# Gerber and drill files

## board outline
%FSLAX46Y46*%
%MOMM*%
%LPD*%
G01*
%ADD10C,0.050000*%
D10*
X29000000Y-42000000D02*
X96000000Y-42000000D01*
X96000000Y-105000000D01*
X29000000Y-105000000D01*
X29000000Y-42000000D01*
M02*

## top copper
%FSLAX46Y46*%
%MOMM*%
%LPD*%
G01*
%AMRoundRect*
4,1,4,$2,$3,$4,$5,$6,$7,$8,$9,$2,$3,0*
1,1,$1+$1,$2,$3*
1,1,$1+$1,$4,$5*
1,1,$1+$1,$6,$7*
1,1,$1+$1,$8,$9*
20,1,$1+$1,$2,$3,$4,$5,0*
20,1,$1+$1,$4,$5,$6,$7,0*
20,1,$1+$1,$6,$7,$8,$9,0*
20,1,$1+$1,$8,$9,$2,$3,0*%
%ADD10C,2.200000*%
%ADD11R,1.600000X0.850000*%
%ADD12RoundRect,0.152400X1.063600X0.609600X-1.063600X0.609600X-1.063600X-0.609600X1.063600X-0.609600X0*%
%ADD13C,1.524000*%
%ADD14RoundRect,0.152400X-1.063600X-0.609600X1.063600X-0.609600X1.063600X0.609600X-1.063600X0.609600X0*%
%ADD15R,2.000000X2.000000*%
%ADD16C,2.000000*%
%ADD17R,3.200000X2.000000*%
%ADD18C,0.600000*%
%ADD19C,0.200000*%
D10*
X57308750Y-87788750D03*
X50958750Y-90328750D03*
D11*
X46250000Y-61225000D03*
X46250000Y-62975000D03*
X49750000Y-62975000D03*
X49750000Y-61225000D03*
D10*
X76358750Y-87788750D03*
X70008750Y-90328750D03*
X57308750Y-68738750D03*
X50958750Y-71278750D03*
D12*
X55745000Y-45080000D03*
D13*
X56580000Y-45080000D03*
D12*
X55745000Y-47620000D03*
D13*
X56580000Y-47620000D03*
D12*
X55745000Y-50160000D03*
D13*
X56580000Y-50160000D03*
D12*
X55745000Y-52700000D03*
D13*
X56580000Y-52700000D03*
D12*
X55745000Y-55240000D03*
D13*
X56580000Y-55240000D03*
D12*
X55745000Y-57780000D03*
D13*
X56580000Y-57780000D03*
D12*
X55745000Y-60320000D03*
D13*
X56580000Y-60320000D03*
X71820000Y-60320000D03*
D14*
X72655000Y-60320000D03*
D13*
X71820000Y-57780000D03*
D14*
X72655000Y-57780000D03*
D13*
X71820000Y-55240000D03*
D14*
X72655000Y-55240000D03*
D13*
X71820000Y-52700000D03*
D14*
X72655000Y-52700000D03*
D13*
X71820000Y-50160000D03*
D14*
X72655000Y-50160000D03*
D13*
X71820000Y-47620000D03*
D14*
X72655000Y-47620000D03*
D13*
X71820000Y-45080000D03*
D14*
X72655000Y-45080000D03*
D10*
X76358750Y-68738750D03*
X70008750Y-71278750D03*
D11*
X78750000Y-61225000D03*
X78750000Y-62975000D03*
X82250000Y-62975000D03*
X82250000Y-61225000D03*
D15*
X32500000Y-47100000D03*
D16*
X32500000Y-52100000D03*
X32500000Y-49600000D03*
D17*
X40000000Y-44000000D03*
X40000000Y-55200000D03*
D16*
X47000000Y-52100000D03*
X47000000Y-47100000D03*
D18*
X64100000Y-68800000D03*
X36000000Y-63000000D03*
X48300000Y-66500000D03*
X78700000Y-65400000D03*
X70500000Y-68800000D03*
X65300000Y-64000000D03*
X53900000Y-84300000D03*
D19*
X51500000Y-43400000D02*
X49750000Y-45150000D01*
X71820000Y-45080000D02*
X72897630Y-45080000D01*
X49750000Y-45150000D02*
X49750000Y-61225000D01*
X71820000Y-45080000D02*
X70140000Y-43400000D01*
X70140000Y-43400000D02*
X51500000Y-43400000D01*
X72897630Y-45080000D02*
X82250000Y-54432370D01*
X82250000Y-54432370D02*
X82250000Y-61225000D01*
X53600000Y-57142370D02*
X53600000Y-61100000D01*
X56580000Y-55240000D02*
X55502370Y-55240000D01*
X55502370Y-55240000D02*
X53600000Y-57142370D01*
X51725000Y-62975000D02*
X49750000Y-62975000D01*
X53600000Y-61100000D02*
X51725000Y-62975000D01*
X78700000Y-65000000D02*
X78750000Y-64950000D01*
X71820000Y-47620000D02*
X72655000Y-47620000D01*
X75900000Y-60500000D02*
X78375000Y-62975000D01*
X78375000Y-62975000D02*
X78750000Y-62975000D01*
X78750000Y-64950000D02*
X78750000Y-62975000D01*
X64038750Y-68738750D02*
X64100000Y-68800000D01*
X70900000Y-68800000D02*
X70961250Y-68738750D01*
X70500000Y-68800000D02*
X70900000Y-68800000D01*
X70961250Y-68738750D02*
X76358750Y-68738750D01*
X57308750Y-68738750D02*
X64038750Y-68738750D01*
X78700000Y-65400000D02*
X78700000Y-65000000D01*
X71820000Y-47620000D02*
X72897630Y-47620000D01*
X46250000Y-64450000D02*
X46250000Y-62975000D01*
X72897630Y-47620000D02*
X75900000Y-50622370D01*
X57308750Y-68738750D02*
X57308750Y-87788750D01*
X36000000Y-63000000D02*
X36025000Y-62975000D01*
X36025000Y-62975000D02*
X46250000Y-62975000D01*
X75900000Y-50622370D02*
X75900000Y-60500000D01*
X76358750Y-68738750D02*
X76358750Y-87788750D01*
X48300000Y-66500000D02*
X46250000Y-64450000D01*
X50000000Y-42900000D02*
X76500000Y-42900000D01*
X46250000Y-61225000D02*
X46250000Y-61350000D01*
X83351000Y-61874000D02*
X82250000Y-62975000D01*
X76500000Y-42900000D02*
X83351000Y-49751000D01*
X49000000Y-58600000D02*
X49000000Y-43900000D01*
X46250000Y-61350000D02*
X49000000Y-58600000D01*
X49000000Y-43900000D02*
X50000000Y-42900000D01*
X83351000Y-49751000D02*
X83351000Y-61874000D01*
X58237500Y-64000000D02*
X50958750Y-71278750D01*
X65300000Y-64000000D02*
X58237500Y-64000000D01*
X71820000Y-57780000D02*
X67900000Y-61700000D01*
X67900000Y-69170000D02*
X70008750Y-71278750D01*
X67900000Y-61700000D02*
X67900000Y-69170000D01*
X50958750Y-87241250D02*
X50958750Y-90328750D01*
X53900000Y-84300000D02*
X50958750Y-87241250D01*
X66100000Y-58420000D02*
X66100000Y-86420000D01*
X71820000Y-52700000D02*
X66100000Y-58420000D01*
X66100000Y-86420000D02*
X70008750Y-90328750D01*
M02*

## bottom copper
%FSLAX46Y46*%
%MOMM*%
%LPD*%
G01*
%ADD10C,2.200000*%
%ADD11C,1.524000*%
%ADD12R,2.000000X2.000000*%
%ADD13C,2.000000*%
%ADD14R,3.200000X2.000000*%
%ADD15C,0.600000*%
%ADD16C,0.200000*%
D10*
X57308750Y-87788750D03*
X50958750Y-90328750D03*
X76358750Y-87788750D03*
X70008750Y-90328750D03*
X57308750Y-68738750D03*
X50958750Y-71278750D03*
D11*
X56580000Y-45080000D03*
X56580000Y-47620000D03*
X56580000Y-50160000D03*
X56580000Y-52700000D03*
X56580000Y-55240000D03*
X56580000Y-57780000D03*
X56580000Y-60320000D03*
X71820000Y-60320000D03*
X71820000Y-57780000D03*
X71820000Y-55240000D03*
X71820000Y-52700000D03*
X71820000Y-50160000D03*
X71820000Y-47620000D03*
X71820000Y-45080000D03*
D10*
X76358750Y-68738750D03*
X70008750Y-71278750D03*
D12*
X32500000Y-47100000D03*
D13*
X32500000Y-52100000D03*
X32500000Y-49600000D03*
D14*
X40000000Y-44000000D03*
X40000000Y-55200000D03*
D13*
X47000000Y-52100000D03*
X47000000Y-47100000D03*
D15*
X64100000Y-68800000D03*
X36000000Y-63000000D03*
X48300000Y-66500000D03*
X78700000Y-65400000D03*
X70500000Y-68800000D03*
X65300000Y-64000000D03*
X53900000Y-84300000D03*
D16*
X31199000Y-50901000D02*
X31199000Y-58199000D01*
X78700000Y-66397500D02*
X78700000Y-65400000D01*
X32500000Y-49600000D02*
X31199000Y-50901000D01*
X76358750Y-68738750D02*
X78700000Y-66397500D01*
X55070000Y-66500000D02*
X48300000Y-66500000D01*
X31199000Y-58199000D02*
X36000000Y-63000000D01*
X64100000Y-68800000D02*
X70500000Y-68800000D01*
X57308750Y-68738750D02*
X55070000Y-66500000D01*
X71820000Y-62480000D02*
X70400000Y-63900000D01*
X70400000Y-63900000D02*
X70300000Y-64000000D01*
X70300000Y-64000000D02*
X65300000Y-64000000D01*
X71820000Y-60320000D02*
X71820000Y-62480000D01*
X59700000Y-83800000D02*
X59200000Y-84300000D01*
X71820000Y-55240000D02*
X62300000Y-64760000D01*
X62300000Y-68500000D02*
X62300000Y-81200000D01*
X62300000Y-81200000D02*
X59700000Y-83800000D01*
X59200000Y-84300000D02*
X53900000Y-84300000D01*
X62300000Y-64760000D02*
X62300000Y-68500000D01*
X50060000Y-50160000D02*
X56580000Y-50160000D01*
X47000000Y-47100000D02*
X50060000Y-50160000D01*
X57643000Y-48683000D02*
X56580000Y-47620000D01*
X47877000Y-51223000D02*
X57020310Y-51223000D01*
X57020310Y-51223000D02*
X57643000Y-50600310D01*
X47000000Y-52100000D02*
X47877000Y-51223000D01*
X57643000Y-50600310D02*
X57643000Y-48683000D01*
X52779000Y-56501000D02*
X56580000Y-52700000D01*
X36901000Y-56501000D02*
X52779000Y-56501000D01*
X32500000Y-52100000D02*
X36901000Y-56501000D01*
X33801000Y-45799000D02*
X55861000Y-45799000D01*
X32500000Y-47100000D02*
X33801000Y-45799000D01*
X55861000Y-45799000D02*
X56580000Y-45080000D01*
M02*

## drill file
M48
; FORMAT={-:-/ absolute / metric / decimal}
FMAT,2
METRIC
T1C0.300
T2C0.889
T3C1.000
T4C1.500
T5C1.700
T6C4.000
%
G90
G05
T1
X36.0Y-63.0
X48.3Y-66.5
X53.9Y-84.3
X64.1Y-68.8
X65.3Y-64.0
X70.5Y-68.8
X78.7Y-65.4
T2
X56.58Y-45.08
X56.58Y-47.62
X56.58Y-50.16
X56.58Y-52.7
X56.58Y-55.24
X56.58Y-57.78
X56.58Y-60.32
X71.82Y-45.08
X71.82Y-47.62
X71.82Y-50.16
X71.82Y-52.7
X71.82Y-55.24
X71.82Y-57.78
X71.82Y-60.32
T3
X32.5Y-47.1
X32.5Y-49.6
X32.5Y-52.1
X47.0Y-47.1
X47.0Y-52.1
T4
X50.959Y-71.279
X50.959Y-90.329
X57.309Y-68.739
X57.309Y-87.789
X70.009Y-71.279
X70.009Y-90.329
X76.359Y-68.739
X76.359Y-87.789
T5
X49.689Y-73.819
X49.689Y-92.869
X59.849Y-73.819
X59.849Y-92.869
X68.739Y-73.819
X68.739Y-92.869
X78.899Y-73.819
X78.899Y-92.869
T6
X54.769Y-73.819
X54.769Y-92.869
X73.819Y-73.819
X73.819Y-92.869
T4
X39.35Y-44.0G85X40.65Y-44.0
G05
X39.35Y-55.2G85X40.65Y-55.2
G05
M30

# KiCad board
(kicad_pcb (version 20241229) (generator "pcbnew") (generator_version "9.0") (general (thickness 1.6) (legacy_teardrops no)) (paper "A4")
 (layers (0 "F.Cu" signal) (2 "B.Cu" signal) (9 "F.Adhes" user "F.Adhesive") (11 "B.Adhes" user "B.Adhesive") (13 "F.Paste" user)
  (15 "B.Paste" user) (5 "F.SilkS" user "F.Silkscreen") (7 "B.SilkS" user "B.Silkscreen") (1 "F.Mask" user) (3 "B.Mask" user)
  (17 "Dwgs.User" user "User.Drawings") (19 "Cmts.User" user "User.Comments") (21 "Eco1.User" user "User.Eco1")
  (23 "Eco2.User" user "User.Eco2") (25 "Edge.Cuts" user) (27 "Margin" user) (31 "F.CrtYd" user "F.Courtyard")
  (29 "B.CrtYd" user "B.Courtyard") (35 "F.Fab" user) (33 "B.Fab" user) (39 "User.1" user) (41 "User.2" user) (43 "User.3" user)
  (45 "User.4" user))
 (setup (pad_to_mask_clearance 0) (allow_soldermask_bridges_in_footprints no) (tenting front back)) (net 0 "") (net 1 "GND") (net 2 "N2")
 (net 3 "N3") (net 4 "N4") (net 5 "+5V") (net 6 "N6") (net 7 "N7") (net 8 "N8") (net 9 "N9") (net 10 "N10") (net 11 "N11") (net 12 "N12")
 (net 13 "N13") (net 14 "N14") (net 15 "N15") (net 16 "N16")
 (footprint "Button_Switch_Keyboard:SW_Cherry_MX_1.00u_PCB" (layer "F.Cu") (at 57.30875 87.78875)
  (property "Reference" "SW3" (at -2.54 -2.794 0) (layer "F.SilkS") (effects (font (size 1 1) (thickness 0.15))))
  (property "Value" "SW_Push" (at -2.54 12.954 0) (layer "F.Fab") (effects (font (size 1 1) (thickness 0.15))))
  (pad "" np_thru_hole circle (at -7.62 5.08) (size 1.7 1.7) (drill 1.7) (layers "*.Cu" "*.Mask"))
  (pad "" np_thru_hole circle (at -2.54 5.08) (size 4 4) (drill 4) (layers "*.Cu" "*.Mask"))
  (pad "" np_thru_hole circle (at 2.54 5.08) (size 1.7 1.7) (drill 1.7) (layers "*.Cu" "*.Mask"))
  (pad "1" thru_hole circle (at 0 0) (size 2.2 2.2) (drill 1.5) (layers "*.Cu" "*.Mask") (remove_unused_layers no) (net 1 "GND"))
  (pad "2" thru_hole circle (at -6.35 2.54) (size 2.2 2.2) (drill 1.5) (layers "*.Cu" "*.Mask") (remove_unused_layers no) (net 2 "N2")))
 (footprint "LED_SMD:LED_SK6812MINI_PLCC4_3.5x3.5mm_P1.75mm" (layer "F.Cu") (at 48 62.1)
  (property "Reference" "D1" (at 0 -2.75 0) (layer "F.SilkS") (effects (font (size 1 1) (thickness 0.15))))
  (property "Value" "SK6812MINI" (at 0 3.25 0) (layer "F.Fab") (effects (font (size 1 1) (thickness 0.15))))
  (pad "1" smd rect (at -1.75 -0.875) (size 1.6 0.85) (layers "F.Cu" "F.Mask" "F.Paste") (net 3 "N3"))
  (pad "2" smd rect (at -1.75 0.875) (size 1.6 0.85) (layers "F.Cu" "F.Mask" "F.Paste") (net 1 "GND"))
  (pad "3" smd rect (at 1.75 0.875) (size 1.6 0.85) (layers "F.Cu" "F.Mask" "F.Paste") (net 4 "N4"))
  (pad "4" smd rect (at 1.75 -0.875) (size 1.6 0.85) (layers "F.Cu" "F.Mask" "F.Paste") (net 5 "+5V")))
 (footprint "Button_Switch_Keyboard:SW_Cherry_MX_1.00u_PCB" (layer "F.Cu") (at 76.35875 87.78875)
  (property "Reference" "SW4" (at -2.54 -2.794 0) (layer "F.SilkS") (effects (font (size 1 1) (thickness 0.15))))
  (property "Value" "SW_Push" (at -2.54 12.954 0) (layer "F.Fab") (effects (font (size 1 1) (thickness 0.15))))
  (pad "" np_thru_hole circle (at -7.62 5.08) (size 1.7 1.7) (drill 1.7) (layers "*.Cu" "*.Mask"))
  (pad "" np_thru_hole circle (at -2.54 5.08) (size 4 4) (drill 4) (layers "*.Cu" "*.Mask"))
  (pad "" np_thru_hole circle (at 2.54 5.08) (size 1.7 1.7) (drill 1.7) (layers "*.Cu" "*.Mask"))
  (pad "1" thru_hole circle (at 0 0) (size 2.2 2.2) (drill 1.5) (layers "*.Cu" "*.Mask") (remove_unused_layers no) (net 1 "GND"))
  (pad "2" thru_hole circle (at -6.35 2.54) (size 2.2 2.2) (drill 1.5) (layers "*.Cu" "*.Mask") (remove_unused_layers no) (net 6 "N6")))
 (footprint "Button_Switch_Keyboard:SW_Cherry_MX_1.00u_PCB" (layer "F.Cu") (at 57.30875 68.73875)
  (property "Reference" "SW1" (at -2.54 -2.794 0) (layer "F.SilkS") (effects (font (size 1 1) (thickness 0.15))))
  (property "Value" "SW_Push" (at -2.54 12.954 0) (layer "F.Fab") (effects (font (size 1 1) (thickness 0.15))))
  (pad "" np_thru_hole circle (at -7.62 5.08) (size 1.7 1.7) (drill 1.7) (layers "*.Cu" "*.Mask"))
  (pad "" np_thru_hole circle (at -2.54 5.08) (size 4 4) (drill 4) (layers "*.Cu" "*.Mask"))
  (pad "" np_thru_hole circle (at 2.54 5.08) (size 1.7 1.7) (drill 1.7) (layers "*.Cu" "*.Mask"))
  (pad "1" thru_hole circle (at 0 0) (size 2.2 2.2) (drill 1.5) (layers "*.Cu" "*.Mask") (remove_unused_layers no) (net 1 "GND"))
  (pad "2" thru_hole circle (at -6.35 2.54) (size 2.2 2.2) (drill 1.5) (layers "*.Cu" "*.Mask") (remove_unused_layers no) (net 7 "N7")))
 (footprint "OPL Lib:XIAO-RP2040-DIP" (layer "F.Cu") (at 64.2 52.7)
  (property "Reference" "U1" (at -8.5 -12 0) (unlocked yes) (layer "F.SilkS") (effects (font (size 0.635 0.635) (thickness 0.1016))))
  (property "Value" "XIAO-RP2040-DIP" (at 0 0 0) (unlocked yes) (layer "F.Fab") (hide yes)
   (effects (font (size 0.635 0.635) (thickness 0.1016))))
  (pad "1" smd roundrect (at -8.455 -7.62 180) (size 2.432 1.524) (layers "F.Cu" "F.Mask") (roundrect_rratio 0.1) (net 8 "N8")
   (thermal_bridge_angle 45))
  (pad "1" thru_hole circle (at -7.62 -7.62 180) (size 1.524 1.524) (drill 0.889) (layers "*.Cu" "*.Mask") (remove_unused_layers no)
   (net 8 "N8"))
  (pad "2" smd roundrect (at -8.455 -5.08 180) (size 2.432 1.524) (layers "F.Cu" "F.Mask") (roundrect_rratio 0.1) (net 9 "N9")
   (thermal_bridge_angle 45))
  (pad "2" thru_hole circle (at -7.62 -5.08 180) (size 1.524 1.524) (drill 0.889) (layers "*.Cu" "*.Mask") (remove_unused_layers no)
   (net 9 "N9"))
  (pad "3" smd roundrect (at -8.455 -2.54 180) (size 2.432 1.524) (layers "F.Cu" "F.Mask") (roundrect_rratio 0.1) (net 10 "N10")
   (thermal_bridge_angle 45))
  (pad "3" thru_hole circle (at -7.62 -2.54 180) (size 1.524 1.524) (drill 0.889) (layers "*.Cu" "*.Mask") (remove_unused_layers no)
   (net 10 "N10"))
  (pad "4" smd roundrect (at -8.455 0 180) (size 2.432 1.524) (layers "F.Cu" "F.Mask") (roundrect_rratio 0.1) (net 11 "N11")
   (thermal_bridge_angle 45))
  (pad "4" thru_hole circle (at -7.62 0 180) (size 1.524 1.524) (drill 0.889) (layers "*.Cu" "*.Mask") (remove_unused_layers no)
   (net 11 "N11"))
  (pad "5" smd roundrect (at -8.455 2.54 180) (size 2.432 1.524) (layers "F.Cu" "F.Mask") (roundrect_rratio 0.1) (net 4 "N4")
   (thermal_bridge_angle 45))
  (pad "5" thru_hole circle (at -7.62 2.54 180) (size 1.524 1.524) (drill 0.889) (layers "*.Cu" "*.Mask") (remove_unused_layers no)
   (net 4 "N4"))
  (pad "6" smd roundrect (at -8.455 5.08 180) (size 2.432 1.524) (layers "F.Cu" "F.Mask") (roundrect_rratio 0.1) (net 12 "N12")
   (thermal_bridge_angle 45))
  (pad "6" thru_hole circle (at -7.62 5.08 180) (size 1.524 1.524) (drill 0.889) (layers "*.Cu" "*.Mask") (remove_unused_layers no)
   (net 12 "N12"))
  (pad "7" smd roundrect (at -8.455 7.62 180) (size 2.432 1.524) (layers "F.Cu" "F.Mask") (roundrect_rratio 0.1) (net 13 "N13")
   (thermal_bridge_angle 45))
  (pad "7" thru_hole circle (at -7.62 7.62 180) (size 1.524 1.524) (drill 0.889) (layers "*.Cu" "*.Mask") (remove_unused_layers no)
   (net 13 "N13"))
  (pad "8" thru_hole circle (at 7.62 7.62) (size 1.524 1.524) (drill 0.889) (layers "*.Cu" "*.Mask") (remove_unused_layers no) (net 7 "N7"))
  (pad "8" smd roundrect (at 8.455 7.62) (size 2.432 1.524) (layers "F.Cu" "F.Mask") (roundrect_rratio 0.1) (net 7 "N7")
   (thermal_bridge_angle 45))
  (pad "9" thru_hole circle (at 7.62 5.08) (size 1.524 1.524) (drill 0.889) (layers "*.Cu" "*.Mask") (remove_unused_layers no)
   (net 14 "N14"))
  (pad "9" smd roundrect (at 8.455 5.08) (size 2.432 1.524) (layers "F.Cu" "F.Mask") (roundrect_rratio 0.1) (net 14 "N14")
   (thermal_bridge_angle 45))
  (pad "10" thru_hole circle (at 7.62 2.54) (size 1.524 1.524) (drill 0.889) (layers "*.Cu" "*.Mask") (remove_unused_layers no) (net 2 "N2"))
  (pad "10" smd roundrect (at 8.455 2.54) (size 2.432 1.524) (layers "F.Cu" "F.Mask") (roundrect_rratio 0.1) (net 2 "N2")
   (thermal_bridge_angle 45))
  (pad "11" thru_hole circle (at 7.62 0) (size 1.524 1.524) (drill 0.889) (layers "*.Cu" "*.Mask") (remove_unused_layers no) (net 6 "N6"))
  (pad "11" smd roundrect (at 8.455 0) (size 2.432 1.524) (layers "F.Cu" "F.Mask") (roundrect_rratio 0.1) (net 6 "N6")
   (thermal_bridge_angle 45))
  (pad "12" thru_hole circle (at 7.62 -2.54) (size 1.524 1.524) (drill 0.889) (layers "*.Cu" "*.Mask") (remove_unused_layers no)
   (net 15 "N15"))
  (pad "12" smd roundrect (at 8.455 -2.54) (size 2.432 1.524) (layers "F.Cu" "F.Mask") (roundrect_rratio 0.1) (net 15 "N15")
   (thermal_bridge_angle 45))
  (pad "13" thru_hole circle (at 7.62 -5.08) (size 1.524 1.524) (drill 0.889) (layers "*.Cu" "*.Mask") (remove_unused_layers no)
   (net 1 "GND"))
  (pad "13" smd roundrect (at 8.455 -5.08) (size 2.432 1.524) (layers "F.Cu" "F.Mask") (roundrect_rratio 0.1) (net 1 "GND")
   (thermal_bridge_angle 45))
  (pad "14" thru_hole circle (at 7.62 -7.62) (size 1.524 1.524) (drill 0.889) (layers "*.Cu" "*.Mask") (remove_unused_layers no)
   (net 5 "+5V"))
  (pad "14" smd roundrect (at 8.455 -7.62) (size 2.432 1.524) (layers "F.Cu" "F.Mask") (roundrect_rratio 0.1) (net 5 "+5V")
   (thermal_bridge_angle 45)))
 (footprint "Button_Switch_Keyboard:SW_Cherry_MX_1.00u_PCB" (layer "F.Cu") (at 76.35875 68.73875)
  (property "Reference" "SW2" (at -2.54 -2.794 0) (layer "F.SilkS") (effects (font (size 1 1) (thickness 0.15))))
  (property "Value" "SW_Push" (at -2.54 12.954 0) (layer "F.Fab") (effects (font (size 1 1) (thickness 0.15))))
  (pad "" np_thru_hole circle (at -7.62 5.08) (size 1.7 1.7) (drill 1.7) (layers "*.Cu" "*.Mask"))
  (pad "" np_thru_hole circle (at -2.54 5.08) (size 4 4) (drill 4) (layers "*.Cu" "*.Mask"))
  (pad "" np_thru_hole circle (at 2.54 5.08) (size 1.7 1.7) (drill 1.7) (layers "*.Cu" "*.Mask"))
  (pad "1" thru_hole circle (at 0 0) (size 2.2 2.2) (drill 1.5) (layers "*.Cu" "*.Mask") (remove_unused_layers no) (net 1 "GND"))
  (pad "2" thru_hole circle (at -6.35 2.54) (size 2.2 2.2) (drill 1.5) (layers "*.Cu" "*.Mask") (remove_unused_layers no) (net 14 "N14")))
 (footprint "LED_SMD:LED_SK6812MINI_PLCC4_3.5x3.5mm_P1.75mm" (layer "F.Cu") (at 80.5 62.1)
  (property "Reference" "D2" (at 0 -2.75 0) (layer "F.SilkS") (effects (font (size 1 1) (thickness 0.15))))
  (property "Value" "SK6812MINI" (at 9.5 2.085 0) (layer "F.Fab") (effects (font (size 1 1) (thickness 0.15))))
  (pad "1" smd rect (at -1.75 -0.875) (size 1.6 0.85) (layers "F.Cu" "F.Mask" "F.Paste") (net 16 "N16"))
  (pad "2" smd rect (at -1.75 0.875) (size 1.6 0.85) (layers "F.Cu" "F.Mask" "F.Paste") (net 1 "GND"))
  (pad "3" smd rect (at 1.75 0.875) (size 1.6 0.85) (layers "F.Cu" "F.Mask" "F.Paste") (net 3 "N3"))
  (pad "4" smd rect (at 1.75 -0.875) (size 1.6 0.85) (layers "F.Cu" "F.Mask" "F.Paste") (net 5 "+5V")))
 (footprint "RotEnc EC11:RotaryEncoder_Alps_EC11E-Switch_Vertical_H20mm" (layer "F.Cu") (at 32.5 47.1)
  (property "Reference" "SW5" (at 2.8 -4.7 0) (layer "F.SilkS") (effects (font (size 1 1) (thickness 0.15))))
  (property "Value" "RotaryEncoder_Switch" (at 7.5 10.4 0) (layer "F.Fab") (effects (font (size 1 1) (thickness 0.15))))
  (pad "A" thru_hole rect (at 0 0) (size 2 2) (drill 1) (layers "*.Cu" "*.Mask") (remove_unused_layers no) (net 8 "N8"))
  (pad "B" thru_hole circle (at 0 5) (size 2 2) (drill 1) (layers "*.Cu" "*.Mask") (remove_unused_layers no) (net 11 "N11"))
  (pad "C" thru_hole circle (at 0 2.5) (size 2 2) (drill 1) (layers "*.Cu" "*.Mask") (remove_unused_layers no) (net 1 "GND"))
  (pad "MP" thru_hole rect (at 7.5 -3.1) (size 3.2 2) (drill oval 2.8 1.5) (layers "*.Cu" "*.Mask") (remove_unused_layers no))
  (pad "MP" thru_hole rect (at 7.5 8.1) (size 3.2 2) (drill oval 2.8 1.5) (layers "*.Cu" "*.Mask") (remove_unused_layers no))
  (pad "S1" thru_hole circle (at 14.5 5) (size 2 2) (drill 1) (layers "*.Cu" "*.Mask") (remove_unused_layers no) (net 9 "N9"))
  (pad "S2" thru_hole circle (at 14.5 0) (size 2 2) (drill 1) (layers "*.Cu" "*.Mask") (remove_unused_layers no) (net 10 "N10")))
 (gr_rect (start 29 42) (end 96 105) (stroke (width 0.05) (type default)) (fill no) (layer "Edge.Cuts"))
 (segment (start 51.5 43.4) (end 49.75 45.15) (width 0.2) (layer "F.Cu") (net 5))
 (segment (start 71.82 45.08) (end 72.89763 45.08) (width 0.2) (layer "F.Cu") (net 5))
 (segment (start 49.75 45.15) (end 49.75 61.225) (width 0.2) (layer "F.Cu") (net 5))
 (segment (start 71.82 45.08) (end 70.14 43.4) (width 0.2) (layer "F.Cu") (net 5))
 (segment (start 70.14 43.4) (end 51.5 43.4) (width 0.2) (layer "F.Cu") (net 5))
 (segment (start 72.89763 45.08) (end 82.25 54.43237) (width 0.2) (layer "F.Cu") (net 5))
 (segment (start 82.25 54.43237) (end 82.25 61.225) (width 0.2) (layer "F.Cu") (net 5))
 (segment (start 53.6 57.14237) (end 53.6 61.1) (width 0.2) (layer "F.Cu") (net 4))
 (segment (start 56.58 55.24) (end 55.50237 55.24) (width 0.2) (layer "F.Cu") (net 4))
 (segment (start 55.50237 55.24) (end 53.6 57.14237) (width 0.2) (layer "F.Cu") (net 4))
 (segment (start 51.725 62.975) (end 49.75 62.975) (width 0.2) (layer "F.Cu") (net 4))
 (segment (start 53.6 61.1) (end 51.725 62.975) (width 0.2) (layer "F.Cu") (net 4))
 (segment (start 78.7 65) (end 78.75 64.95) (width 0.2) (layer "F.Cu") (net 1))
 (segment (start 71.82 47.62) (end 72.655 47.62) (width 0.2) (layer "F.Cu") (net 1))
 (segment (start 75.9 60.5) (end 78.375 62.975) (width 0.2) (layer "F.Cu") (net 1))
 (segment (start 78.375 62.975) (end 78.75 62.975) (width 0.2) (layer "F.Cu") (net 1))
 (segment (start 78.75 64.95) (end 78.75 62.975) (width 0.2) (layer "F.Cu") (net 1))
 (segment (start 64.03875 68.73875) (end 64.1 68.8) (width 0.2) (layer "F.Cu") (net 1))
 (segment (start 70.9 68.8) (end 70.96125 68.73875) (width 0.2) (layer "F.Cu") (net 1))
 (segment (start 70.5 68.8) (end 70.9 68.8) (width 0.2) (layer "F.Cu") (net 1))
 (segment (start 70.96125 68.73875) (end 76.35875 68.73875) (width 0.2) (layer "F.Cu") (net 1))
 (segment (start 57.30875 68.73875) (end 64.03875 68.73875) (width 0.2) (layer "F.Cu") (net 1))
 (segment (start 78.7 65.4) (end 78.7 65) (width 0.2) (layer "F.Cu") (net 1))
 (segment (start 71.82 47.62) (end 72.89763 47.62) (width 0.2) (layer "F.Cu") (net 1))
 (segment (start 46.25 64.45) (end 46.25 62.975) (width 0.2) (layer "F.Cu") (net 1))
 (segment (start 72.89763 47.62) (end 75.9 50.62237) (width 0.2) (layer "F.Cu") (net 1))
 (segment (start 57.30875 68.73875) (end 57.30875 87.78875) (width 0.2) (layer "F.Cu") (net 1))
 (segment (start 36 63) (end 36.025 62.975) (width 0.2) (layer "F.Cu") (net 1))
 (segment (start 36.025 62.975) (end 46.25 62.975) (width 0.2) (layer "F.Cu") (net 1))
 (segment (start 75.9 50.62237) (end 75.9 60.5) (width 0.2) (layer "F.Cu") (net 1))
 (segment (start 76.35875 68.73875) (end 76.35875 87.78875) (width 0.2) (layer "F.Cu") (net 1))
 (segment (start 48.3 66.5) (end 46.25 64.45) (width 0.2) (layer "F.Cu") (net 1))
 (via (at 64.1 68.8) (size 0.6) (drill 0.3) (layers "F.Cu" "B.Cu") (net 1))
 (via (at 36 63) (size 0.6) (drill 0.3) (layers "F.Cu" "B.Cu") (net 1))
 (via (at 48.3 66.5) (size 0.6) (drill 0.3) (layers "F.Cu" "B.Cu") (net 1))
 (via (at 78.7 65.4) (size 0.6) (drill 0.3) (layers "F.Cu" "B.Cu") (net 1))
 (via (at 70.5 68.8) (size 0.6) (drill 0.3) (layers "F.Cu" "B.Cu") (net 1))
 (segment (start 31.199 50.901) (end 31.199 58.199) (width 0.2) (layer "B.Cu") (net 1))
 (segment (start 78.7 66.3975) (end 78.7 65.4) (width 0.2) (layer "B.Cu") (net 1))
 (segment (start 32.5 49.6) (end 31.199 50.901) (width 0.2) (layer "B.Cu") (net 1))
 (segment (start 76.35875 68.73875) (end 78.7 66.3975) (width 0.2) (layer "B.Cu") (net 1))
 (segment (start 55.07 66.5) (end 48.3 66.5) (width 0.2) (layer "B.Cu") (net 1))
 (segment (start 31.199 58.199) (end 36 63) (width 0.2) (layer "B.Cu") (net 1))
 (segment (start 64.1 68.8) (end 70.5 68.8) (width 0.2) (layer "B.Cu") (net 1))
 (segment (start 57.30875 68.73875) (end 55.07 66.5) (width 0.2) (layer "B.Cu") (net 1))
 (segment (start 50 42.9) (end 76.5 42.9) (width 0.2) (layer "F.Cu") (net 3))
 (segment (start 46.25 61.225) (end 46.25 61.35) (width 0.2) (layer "F.Cu") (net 3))
 (segment (start 83.351 61.874) (end 82.25 62.975) (width 0.2) (layer "F.Cu") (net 3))
 (segment (start 76.5 42.9) (end 83.351 49.751) (width 0.2) (layer "F.Cu") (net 3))
 (segment (start 49 58.6) (end 49 43.9) (width 0.2) (layer "F.Cu") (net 3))
 (segment (start 46.25 61.35) (end 49 58.6) (width 0.2) (layer "F.Cu") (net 3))
 (segment (start 49 43.9) (end 50 42.9) (width 0.2) (layer "F.Cu") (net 3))
 (segment (start 83.351 49.751) (end 83.351 61.874) (width 0.2) (layer "F.Cu") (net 3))
 (segment (start 58.2375 64) (end 50.95875 71.27875) (width 0.2) (layer "F.Cu") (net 7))
 (segment (start 65.3 64) (end 58.2375 64) (width 0.2) (layer "F.Cu") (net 7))
 (via (at 65.3 64) (size 0.6) (drill 0.3) (layers "F.Cu" "B.Cu") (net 7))
 (segment (start 71.82 62.48) (end 70.4 63.9) (width 0.2) (layer "B.Cu") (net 7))
 (segment (start 70.4 63.9) (end 70.3 64) (width 0.2) (layer "B.Cu") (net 7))
 (segment (start 70.3 64) (end 65.3 64) (width 0.2) (layer "B.Cu") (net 7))
 (segment (start 71.82 60.32) (end 71.82 62.48) (width 0.2) (layer "B.Cu") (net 7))
 (segment (start 71.82 57.78) (end 67.9 61.7) (width 0.2) (layer "F.Cu") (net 14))
 (segment (start 67.9 69.17) (end 70.00875 71.27875) (width 0.2) (layer "F.Cu") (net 14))
 (segment (start 67.9 61.7) (end 67.9 69.17) (width 0.2) (layer "F.Cu") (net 14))
 (segment (start 50.95875 87.24125) (end 50.95875 90.32875) (width 0.2) (layer "F.Cu") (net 2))
 (segment (start 53.9 84.3) (end 50.95875 87.24125) (width 0.2) (layer "F.Cu") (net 2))
 (via (at 53.9 84.3) (size 0.6) (drill 0.3) (layers "F.Cu" "B.Cu") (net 2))
 (segment (start 59.7 83.8) (end 59.2 84.3) (width 0.2) (layer "B.Cu") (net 2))
 (segment (start 71.82 55.24) (end 62.3 64.76) (width 0.2) (layer "B.Cu") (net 2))
 (segment (start 62.3 68.5) (end 62.3 81.2) (width 0.2) (layer "B.Cu") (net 2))
 (segment (start 62.3 81.2) (end 59.7 83.8) (width 0.2) (layer "B.Cu") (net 2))
 (segment (start 59.2 84.3) (end 53.9 84.3) (width 0.2) (layer "B.Cu") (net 2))
 (segment (start 62.3 64.76) (end 62.3 68.5) (width 0.2) (layer "B.Cu") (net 2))
 (segment (start 66.1 58.42) (end 66.1 86.42) (width 0.2) (layer "F.Cu") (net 6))
 (segment (start 71.82 52.7) (end 66.1 58.42) (width 0.2) (layer "F.Cu") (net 6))
 (segment (start 66.1 86.42) (end 70.00875 90.32875) (width 0.2) (layer "F.Cu") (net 6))
 (segment (start 50.06 50.16) (end 56.58 50.16) (width 0.2) (layer "B.Cu") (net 10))
 (segment (start 47 47.1) (end 50.06 50.16) (width 0.2) (layer "B.Cu") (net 10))
 (segment (start 57.643 48.683) (end 56.58 47.62) (width 0.2) (layer "B.Cu") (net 9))
 (segment (start 47.877 51.223) (end 57.02031 51.223) (width 0.2) (layer "B.Cu") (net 9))
 (segment (start 57.02031 51.223) (end 57.643 50.60031) (width 0.2) (layer "B.Cu") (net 9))
 (segment (start 47 52.1) (end 47.877 51.223) (width 0.2) (layer "B.Cu") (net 9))
 (segment (start 57.643 50.60031) (end 57.643 48.683) (width 0.2) (layer "B.Cu") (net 9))
 (segment (start 52.779 56.501) (end 56.58 52.7) (width 0.2) (layer "B.Cu") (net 11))
 (segment (start 36.901 56.501) (end 52.779 56.501) (width 0.2) (layer "B.Cu") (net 11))
 (segment (start 32.5 52.1) (end 36.901 56.501) (width 0.2) (layer "B.Cu") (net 11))
 (segment (start 33.801 45.799) (end 55.861 45.799) (width 0.2) (layer "B.Cu") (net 8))
 (segment (start 32.5 47.1) (end 33.801 45.799) (width 0.2) (layer "B.Cu") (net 8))
 (segment (start 55.861 45.799) (end 56.58 45.08) (width 0.2) (layer "B.Cu") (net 8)))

